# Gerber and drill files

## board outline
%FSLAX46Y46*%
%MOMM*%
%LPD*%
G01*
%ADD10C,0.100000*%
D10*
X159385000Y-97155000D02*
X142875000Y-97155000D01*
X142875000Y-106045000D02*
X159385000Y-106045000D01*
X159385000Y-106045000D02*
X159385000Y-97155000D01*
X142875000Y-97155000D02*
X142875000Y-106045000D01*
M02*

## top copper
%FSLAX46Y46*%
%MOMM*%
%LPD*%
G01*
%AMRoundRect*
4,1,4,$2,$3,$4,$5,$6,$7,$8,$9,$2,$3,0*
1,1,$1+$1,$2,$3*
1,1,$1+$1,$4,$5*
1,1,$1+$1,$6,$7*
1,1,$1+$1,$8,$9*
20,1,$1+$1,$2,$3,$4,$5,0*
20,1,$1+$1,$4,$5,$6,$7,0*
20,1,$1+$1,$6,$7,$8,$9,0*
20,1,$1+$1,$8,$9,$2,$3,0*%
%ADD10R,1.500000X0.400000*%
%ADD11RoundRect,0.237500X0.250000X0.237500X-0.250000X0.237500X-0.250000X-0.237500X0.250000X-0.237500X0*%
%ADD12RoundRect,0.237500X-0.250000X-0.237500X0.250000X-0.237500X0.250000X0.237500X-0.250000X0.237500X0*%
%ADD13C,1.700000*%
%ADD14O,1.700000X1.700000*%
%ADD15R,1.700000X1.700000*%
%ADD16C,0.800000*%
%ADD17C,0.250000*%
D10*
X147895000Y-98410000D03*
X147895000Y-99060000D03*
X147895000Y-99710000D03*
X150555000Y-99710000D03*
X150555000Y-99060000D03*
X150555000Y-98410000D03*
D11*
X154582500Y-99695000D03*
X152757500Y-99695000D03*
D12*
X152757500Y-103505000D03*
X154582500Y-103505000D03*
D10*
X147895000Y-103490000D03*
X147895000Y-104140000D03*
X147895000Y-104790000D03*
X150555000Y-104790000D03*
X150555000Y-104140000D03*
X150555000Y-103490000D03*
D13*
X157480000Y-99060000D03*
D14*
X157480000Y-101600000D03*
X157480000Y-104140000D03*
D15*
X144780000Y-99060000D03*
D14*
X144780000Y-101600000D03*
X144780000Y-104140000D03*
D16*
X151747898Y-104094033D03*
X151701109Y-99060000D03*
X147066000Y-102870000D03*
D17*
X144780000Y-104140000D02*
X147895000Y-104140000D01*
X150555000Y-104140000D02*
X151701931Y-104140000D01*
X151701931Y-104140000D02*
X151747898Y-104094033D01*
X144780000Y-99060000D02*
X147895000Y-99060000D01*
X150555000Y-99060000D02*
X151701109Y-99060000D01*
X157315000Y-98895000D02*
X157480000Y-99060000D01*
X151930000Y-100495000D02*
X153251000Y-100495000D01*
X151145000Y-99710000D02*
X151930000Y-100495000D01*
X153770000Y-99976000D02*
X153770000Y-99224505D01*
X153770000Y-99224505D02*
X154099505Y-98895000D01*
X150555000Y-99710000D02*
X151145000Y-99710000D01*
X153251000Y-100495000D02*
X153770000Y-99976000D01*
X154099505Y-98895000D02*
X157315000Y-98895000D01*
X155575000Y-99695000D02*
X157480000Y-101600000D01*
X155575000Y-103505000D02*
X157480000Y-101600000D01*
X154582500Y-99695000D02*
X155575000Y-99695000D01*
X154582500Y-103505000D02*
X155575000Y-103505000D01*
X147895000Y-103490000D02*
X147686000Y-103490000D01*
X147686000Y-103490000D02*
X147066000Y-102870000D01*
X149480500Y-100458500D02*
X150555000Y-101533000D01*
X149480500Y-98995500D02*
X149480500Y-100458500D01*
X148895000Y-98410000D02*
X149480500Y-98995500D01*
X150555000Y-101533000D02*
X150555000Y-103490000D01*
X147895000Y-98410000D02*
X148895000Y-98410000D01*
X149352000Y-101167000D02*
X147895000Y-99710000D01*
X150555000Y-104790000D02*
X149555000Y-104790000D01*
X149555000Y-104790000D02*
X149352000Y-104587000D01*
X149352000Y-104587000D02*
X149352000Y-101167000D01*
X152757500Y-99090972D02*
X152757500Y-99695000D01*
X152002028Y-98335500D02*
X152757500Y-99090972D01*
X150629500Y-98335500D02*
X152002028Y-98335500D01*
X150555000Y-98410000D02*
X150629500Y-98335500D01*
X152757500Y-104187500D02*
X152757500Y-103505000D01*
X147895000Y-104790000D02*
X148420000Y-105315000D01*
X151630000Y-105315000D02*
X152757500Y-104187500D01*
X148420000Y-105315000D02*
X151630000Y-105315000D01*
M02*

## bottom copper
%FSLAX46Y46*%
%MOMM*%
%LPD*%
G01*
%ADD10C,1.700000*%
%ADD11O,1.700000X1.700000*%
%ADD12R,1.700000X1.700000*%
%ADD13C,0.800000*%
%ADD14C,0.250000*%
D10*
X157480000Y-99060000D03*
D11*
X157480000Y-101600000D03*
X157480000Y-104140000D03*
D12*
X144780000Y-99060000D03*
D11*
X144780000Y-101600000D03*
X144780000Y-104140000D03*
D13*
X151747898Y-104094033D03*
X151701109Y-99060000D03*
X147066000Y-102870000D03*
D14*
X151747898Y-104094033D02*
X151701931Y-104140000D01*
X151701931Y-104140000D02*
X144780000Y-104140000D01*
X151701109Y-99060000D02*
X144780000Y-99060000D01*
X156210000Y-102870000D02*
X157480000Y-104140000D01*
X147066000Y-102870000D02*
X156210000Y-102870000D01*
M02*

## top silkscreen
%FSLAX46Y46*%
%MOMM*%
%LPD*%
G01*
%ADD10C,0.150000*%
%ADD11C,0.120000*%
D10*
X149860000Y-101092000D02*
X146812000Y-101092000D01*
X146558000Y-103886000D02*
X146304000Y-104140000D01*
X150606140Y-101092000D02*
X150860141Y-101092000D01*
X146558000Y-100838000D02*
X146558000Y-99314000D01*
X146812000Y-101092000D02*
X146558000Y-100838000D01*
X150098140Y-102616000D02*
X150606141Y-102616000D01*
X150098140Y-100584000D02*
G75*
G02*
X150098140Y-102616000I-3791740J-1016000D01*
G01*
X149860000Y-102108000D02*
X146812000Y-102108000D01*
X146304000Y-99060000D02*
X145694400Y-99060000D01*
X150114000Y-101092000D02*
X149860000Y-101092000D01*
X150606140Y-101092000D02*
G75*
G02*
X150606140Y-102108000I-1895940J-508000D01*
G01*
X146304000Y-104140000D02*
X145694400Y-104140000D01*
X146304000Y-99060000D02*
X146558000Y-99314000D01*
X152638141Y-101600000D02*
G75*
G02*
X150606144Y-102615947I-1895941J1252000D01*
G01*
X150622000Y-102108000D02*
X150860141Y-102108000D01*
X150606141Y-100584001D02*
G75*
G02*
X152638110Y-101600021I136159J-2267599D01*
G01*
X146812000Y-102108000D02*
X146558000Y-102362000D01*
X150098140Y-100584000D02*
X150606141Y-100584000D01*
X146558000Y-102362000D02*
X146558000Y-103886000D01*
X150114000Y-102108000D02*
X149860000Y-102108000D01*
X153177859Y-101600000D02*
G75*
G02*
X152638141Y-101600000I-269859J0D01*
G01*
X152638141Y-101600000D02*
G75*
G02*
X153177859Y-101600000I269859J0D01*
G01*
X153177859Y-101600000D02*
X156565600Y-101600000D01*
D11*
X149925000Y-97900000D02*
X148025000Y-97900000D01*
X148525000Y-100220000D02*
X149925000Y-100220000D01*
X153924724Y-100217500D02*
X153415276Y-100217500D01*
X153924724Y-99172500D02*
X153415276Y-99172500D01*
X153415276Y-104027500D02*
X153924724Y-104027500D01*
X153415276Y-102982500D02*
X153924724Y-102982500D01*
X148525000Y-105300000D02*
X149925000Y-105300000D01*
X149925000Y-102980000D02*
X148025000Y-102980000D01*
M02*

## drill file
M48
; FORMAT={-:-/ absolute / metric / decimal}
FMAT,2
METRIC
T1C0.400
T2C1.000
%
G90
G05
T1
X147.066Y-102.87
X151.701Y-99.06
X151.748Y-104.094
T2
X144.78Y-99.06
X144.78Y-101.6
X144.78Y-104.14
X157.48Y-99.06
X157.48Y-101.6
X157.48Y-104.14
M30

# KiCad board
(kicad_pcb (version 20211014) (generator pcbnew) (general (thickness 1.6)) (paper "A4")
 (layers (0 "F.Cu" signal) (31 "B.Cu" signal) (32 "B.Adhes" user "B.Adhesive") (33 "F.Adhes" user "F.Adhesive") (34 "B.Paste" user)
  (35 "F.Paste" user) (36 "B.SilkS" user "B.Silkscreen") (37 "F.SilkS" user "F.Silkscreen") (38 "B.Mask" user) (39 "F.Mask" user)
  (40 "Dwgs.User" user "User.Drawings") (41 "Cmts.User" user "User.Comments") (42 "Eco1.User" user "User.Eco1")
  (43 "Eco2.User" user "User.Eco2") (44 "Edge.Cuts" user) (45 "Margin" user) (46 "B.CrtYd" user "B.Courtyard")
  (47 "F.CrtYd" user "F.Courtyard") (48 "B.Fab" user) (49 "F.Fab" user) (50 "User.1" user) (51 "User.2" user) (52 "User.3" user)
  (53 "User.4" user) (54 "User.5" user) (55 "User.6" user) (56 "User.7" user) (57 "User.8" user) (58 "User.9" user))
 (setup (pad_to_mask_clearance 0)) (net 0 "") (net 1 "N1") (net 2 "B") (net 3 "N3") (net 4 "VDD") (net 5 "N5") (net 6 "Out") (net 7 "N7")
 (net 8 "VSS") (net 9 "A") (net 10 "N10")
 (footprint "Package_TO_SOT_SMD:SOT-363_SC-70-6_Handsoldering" (layer "F.Cu") (at 149.225 99.06)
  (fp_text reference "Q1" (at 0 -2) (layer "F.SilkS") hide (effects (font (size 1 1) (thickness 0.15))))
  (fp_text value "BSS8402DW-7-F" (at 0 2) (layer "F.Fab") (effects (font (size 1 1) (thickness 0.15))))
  (fp_line (start 0.7 -1.16) (end -1.2 -1.16) (layer "F.SilkS") (width 0.12))
  (fp_line (start -0.7 1.16) (end 0.7 1.16) (layer "F.SilkS") (width 0.12))
  (pad "1" smd rect (at -1.33 -0.65) (size 1.5 0.4) (layers "F.Cu" "F.Paste" "F.Mask") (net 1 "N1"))
  (pad "2" smd rect (at -1.33 0) (size 1.5 0.4) (layers "F.Cu" "F.Paste" "F.Mask") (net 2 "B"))
  (pad "3" smd rect (at -1.33 0.65) (size 1.5 0.4) (layers "F.Cu" "F.Paste" "F.Mask") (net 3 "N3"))
  (pad "4" smd rect (at 1.33 0.65) (size 1.5 0.4) (layers "F.Cu" "F.Paste" "F.Mask") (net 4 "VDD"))
  (pad "5" smd rect (at 1.33 0) (size 1.5 0.4) (layers "F.Cu" "F.Paste" "F.Mask") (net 2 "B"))
  (pad "6" smd rect (at 1.33 -0.65) (size 1.5 0.4) (layers "F.Cu" "F.Paste" "F.Mask") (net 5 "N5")))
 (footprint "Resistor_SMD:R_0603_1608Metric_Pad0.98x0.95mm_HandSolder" (layer "F.Cu") (at 153.67 99.695 180)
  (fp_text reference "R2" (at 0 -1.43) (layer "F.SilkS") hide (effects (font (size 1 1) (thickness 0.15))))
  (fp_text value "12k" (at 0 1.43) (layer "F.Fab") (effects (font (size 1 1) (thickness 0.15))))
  (fp_line (start -0.254724 -0.5225) (end 0.254724 -0.5225) (layer "F.SilkS") (width 0.12))
  (fp_line (start -0.254724 0.5225) (end 0.254724 0.5225) (layer "F.SilkS") (width 0.12))
  (pad "1" smd roundrect (at -0.9125 0 180) (size 0.975 0.95) (layers "F.Cu" "F.Paste" "F.Mask") (roundrect_rratio 0.25) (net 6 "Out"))
  (pad "2" smd roundrect (at 0.9125 0 180) (size 0.975 0.95) (layers "F.Cu" "F.Paste" "F.Mask") (roundrect_rratio 0.25) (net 5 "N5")))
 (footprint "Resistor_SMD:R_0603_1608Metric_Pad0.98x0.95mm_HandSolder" (layer "F.Cu") (at 153.67 103.505)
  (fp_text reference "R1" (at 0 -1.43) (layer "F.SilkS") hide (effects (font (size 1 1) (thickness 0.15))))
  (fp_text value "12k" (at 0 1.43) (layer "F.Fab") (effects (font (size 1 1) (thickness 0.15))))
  (fp_line (start -0.254724 0.5225) (end 0.254724 0.5225) (layer "F.SilkS") (width 0.12))
  (fp_line (start -0.254724 -0.5225) (end 0.254724 -0.5225) (layer "F.SilkS") (width 0.12))
  (pad "1" smd roundrect (at -0.9125 0) (size 0.975 0.95) (layers "F.Cu" "F.Paste" "F.Mask") (roundrect_rratio 0.25) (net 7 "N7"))
  (pad "2" smd roundrect (at 0.9125 0) (size 0.975 0.95) (layers "F.Cu" "F.Paste" "F.Mask") (roundrect_rratio 0.25) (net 6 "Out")))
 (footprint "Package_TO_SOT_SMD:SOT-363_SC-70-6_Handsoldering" (layer "F.Cu") (at 149.225 104.14)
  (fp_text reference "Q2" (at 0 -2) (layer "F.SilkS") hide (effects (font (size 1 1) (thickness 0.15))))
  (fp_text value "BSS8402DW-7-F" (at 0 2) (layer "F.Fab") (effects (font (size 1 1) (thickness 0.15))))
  (fp_line (start -0.7 1.16) (end 0.7 1.16) (layer "F.SilkS") (width 0.12))
  (fp_line (start 0.7 -1.16) (end -1.2 -1.16) (layer "F.SilkS") (width 0.12))
  (pad "1" smd rect (at -1.33 -0.65) (size 1.5 0.4) (layers "F.Cu" "F.Paste" "F.Mask") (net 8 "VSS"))
  (pad "2" smd rect (at -1.33 0) (size 1.5 0.4) (layers "F.Cu" "F.Paste" "F.Mask") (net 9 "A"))
  (pad "3" smd rect (at -1.33 0.65) (size 1.5 0.4) (layers "F.Cu" "F.Paste" "F.Mask") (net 7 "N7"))
  (pad "4" smd rect (at 1.33 0.65) (size 1.5 0.4) (layers "F.Cu" "F.Paste" "F.Mask") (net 3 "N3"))
  (pad "5" smd rect (at 1.33 0) (size 1.5 0.4) (layers "F.Cu" "F.Paste" "F.Mask") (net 9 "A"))
  (pad "6" smd rect (at 1.33 -0.65) (size 1.5 0.4) (layers "F.Cu" "F.Paste" "F.Mask") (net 1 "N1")))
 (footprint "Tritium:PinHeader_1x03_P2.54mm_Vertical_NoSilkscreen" (layer "F.Cu") (at 157.48 99.06)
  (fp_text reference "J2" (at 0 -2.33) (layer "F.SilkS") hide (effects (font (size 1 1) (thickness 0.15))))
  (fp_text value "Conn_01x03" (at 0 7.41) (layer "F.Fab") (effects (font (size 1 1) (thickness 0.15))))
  (pad "1" thru_hole circle (at 0 0) (size 1.7 1.7) (drill 1) (layers *.Cu *.Mask) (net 4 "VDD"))
  (pad "2" thru_hole oval (at 0 2.54) (size 1.7 1.7) (drill 1) (layers *.Cu *.Mask) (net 6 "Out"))
  (pad "3" thru_hole oval (at 0 5.08) (size 1.7 1.7) (drill 1) (layers *.Cu *.Mask) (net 8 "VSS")))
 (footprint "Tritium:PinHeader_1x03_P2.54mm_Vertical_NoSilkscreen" (layer "F.Cu") (at 144.78 99.06)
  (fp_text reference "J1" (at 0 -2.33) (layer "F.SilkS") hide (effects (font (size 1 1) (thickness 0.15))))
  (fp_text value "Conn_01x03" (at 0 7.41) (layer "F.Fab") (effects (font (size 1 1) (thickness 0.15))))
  (pad "1" thru_hole rect (at 0 0) (size 1.7 1.7) (drill 1) (layers *.Cu *.Mask) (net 2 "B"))
  (pad "2" thru_hole oval (at 0 2.54) (size 1.7 1.7) (drill 1) (layers *.Cu *.Mask) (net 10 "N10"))
  (pad "3" thru_hole oval (at 0 5.08) (size 1.7 1.7) (drill 1) (layers *.Cu *.Mask) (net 9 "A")))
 (gr_line (start 149.86 101.092) (end 146.812 101.092) (layer "F.SilkS") (width 0.15))
 (gr_line (start 146.558 103.886) (end 146.304 104.14) (layer "F.SilkS") (width 0.15))
 (gr_line (start 150.60614 101.092) (end 150.860141 101.092) (layer "F.SilkS") (width 0.15))
 (gr_line (start 146.558 100.838) (end 146.558 99.314) (layer "F.SilkS") (width 0.15))
 (gr_line (start 146.812 101.092) (end 146.558 100.838) (layer "F.SilkS") (width 0.15))
 (gr_line (start 150.09814 102.616) (end 150.606141 102.616) (layer "F.SilkS") (width 0.15))
 (gr_arc (start 150.09814 100.584) (mid 150.2319 101.6) (end 150.09814 102.616) (layer "F.SilkS") (width 0.15))
 (gr_line (start 149.86 102.108) (end 146.812 102.108) (layer "F.SilkS") (width 0.15))
 (gr_line (start 146.304 99.06) (end 145.6944 99.06) (layer "F.SilkS") (width 0.15))
 (gr_line (start 150.114 101.092) (end 149.86 101.092) (layer "F.SilkS") (width 0.15))
 (gr_arc (start 150.60614 101.092) (mid 150.673017 101.6) (end 150.60614 102.108) (layer "F.SilkS") (width 0.15))
 (gr_line (start 146.304 104.14) (end 145.6944 104.14) (layer "F.SilkS") (width 0.15))
 (gr_line (start 146.304 99.06) (end 146.558 99.314) (layer "F.SilkS") (width 0.15))
 (gr_arc (start 152.638141 101.6) (mid 151.758253 102.380208) (end 150.606141 102.616) (layer "F.SilkS") (width 0.15))
 (gr_line (start 150.622 102.108) (end 150.860141 102.108) (layer "F.SilkS") (width 0.15))
 (gr_arc (start 150.606141 100.584001) (mid 151.758276 100.819746) (end 152.638141 101.6) (layer "F.SilkS") (width 0.15))
 (gr_line (start 146.812 102.108) (end 146.558 102.362) (layer "F.SilkS") (width 0.15))
 (gr_line (start 150.09814 100.584) (end 150.606141 100.584) (layer "F.SilkS") (width 0.15))
 (gr_line (start 146.558 102.362) (end 146.558 103.886) (layer "F.SilkS") (width 0.15))
 (gr_line (start 150.114 102.108) (end 149.86 102.108) (layer "F.SilkS") (width 0.15))
 (gr_circle (center 152.908 101.6) (end 152.638141 101.6) (layer "F.SilkS") (width 0.15) (fill none))
 (gr_line (start 153.177859 101.6) (end 156.5656 101.6) (layer "F.SilkS") (width 0.15))
 (gr_line (start 159.385 97.155) (end 142.875 97.155) (layer "Edge.Cuts") (width 0.1))
 (gr_line (start 142.875 106.045) (end 159.385 106.045) (layer "Edge.Cuts") (width 0.1))
 (gr_line (start 159.385 106.045) (end 159.385 97.155) (layer "Edge.Cuts") (width 0.1))
 (gr_line (start 142.875 97.155) (end 142.875 106.045) (layer "Edge.Cuts") (width 0.1))
 (segment (start 144.78 104.14) (end 147.895 104.14) (width 0.25) (layer "F.Cu") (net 9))
 (segment (start 150.555 104.14) (end 151.701931 104.14) (width 0.25) (layer "F.Cu") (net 9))
 (segment (start 151.701931 104.14) (end 151.747898 104.094033) (width 0.25) (layer "F.Cu") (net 9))
 (via (at 151.747898 104.094033) (size 0.8) (drill 0.4) (layers "F.Cu" "B.Cu") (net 9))
 (segment (start 151.747898 104.094033) (end 151.701931 104.14) (width 0.25) (layer "B.Cu") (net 9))
 (segment (start 151.701931 104.14) (end 144.78 104.14) (width 0.25) (layer "B.Cu") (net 9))
 (segment (start 144.78 99.06) (end 147.895 99.06) (width 0.25) (layer "F.Cu") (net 2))
 (segment (start 150.555 99.06) (end 151.701109 99.06) (width 0.25) (layer "F.Cu") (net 2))
 (via (at 151.701109 99.06) (size 0.8) (drill 0.4) (layers "F.Cu" "B.Cu") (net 2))
 (segment (start 151.701109 99.06) (end 144.78 99.06) (width 0.25) (layer "B.Cu") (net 2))
 (segment (start 157.315 98.895) (end 157.48 99.06) (width 0.25) (layer "F.Cu") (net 4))
 (segment (start 151.93 100.495) (end 153.251 100.495) (width 0.25) (layer "F.Cu") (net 4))
 (segment (start 151.145 99.71) (end 151.93 100.495) (width 0.25) (layer "F.Cu") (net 4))
 (segment (start 153.77 99.976) (end 153.77 99.224505) (width 0.25) (layer "F.Cu") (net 4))
 (segment (start 153.77 99.224505) (end 154.099505 98.895) (width 0.25) (layer "F.Cu") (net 4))
 (segment (start 150.555 99.71) (end 151.145 99.71) (width 0.25) (layer "F.Cu") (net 4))
 (segment (start 153.251 100.495) (end 153.77 99.976) (width 0.25) (layer "F.Cu") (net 4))
 (segment (start 154.099505 98.895) (end 157.315 98.895) (width 0.25) (layer "F.Cu") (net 4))
 (segment (start 155.575 99.695) (end 157.48 101.6) (width 0.25) (layer "F.Cu") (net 6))
 (segment (start 155.575 103.505) (end 157.48 101.6) (width 0.25) (layer "F.Cu") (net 6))
 (segment (start 154.5825 99.695) (end 155.575 99.695) (width 0.25) (layer "F.Cu") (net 6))
 (segment (start 154.5825 103.505) (end 155.575 103.505) (width 0.25) (layer "F.Cu") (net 6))
 (segment (start 147.895 103.49) (end 147.686 103.49) (width 0.25) (layer "F.Cu") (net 8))
 (segment (start 147.686 103.49) (end 147.066 102.87) (width 0.25) (layer "F.Cu") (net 8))
 (via (at 147.066 102.87) (size 0.8) (drill 0.4) (layers "F.Cu" "B.Cu") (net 8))
 (segment (start 156.21 102.87) (end 157.48 104.14) (width 0.25) (layer "B.Cu") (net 8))
 (segment (start 147.066 102.87) (end 156.21 102.87) (width 0.25) (layer "B.Cu") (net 8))
 (segment (start 149.4805 100.4585) (end 150.555 101.533) (width 0.25) (layer "F.Cu") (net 1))
 (segment (start 149.4805 98.9955) (end 149.4805 100.4585) (width 0.25) (layer "F.Cu") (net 1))
 (segment (start 148.895 98.41) (end 149.4805 98.9955) (width 0.25) (layer "F.Cu") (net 1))
 (segment (start 150.555 101.533) (end 150.555 103.49) (width 0.25) (layer "F.Cu") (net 1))
 (segment (start 147.895 98.41) (end 148.895 98.41) (width 0.25) (layer "F.Cu") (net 1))
 (segment (start 149.352 101.167) (end 147.895 99.71) (width 0.25) (layer "F.Cu") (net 3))
 (segment (start 150.555 104.79) (end 149.555 104.79) (width 0.25) (layer "F.Cu") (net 3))
 (segment (start 149.555 104.79) (end 149.352 104.587) (width 0.25) (layer "F.Cu") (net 3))
 (segment (start 149.352 104.587) (end 149.352 101.167) (width 0.25) (layer "F.Cu") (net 3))
 (segment (start 152.7575 99.090972) (end 152.7575 99.695) (width 0.25) (layer "F.Cu") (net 5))
 (segment (start 152.002028 98.3355) (end 152.7575 99.090972) (width 0.25) (layer "F.Cu") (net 5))
 (segment (start 150.6295 98.3355) (end 152.002028 98.3355) (width 0.25) (layer "F.Cu") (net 5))
 (segment (start 150.555 98.41) (end 150.6295 98.3355) (width 0.25) (layer "F.Cu") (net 5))
 (segment (start 152.7575 104.1875) (end 152.7575 103.505) (width 0.25) (layer "F.Cu") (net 7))
 (segment (start 147.895 104.79) (end 148.42 105.315) (width 0.25) (layer "F.Cu") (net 7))
 (segment (start 151.63 105.315) (end 152.7575 104.1875) (width 0.25) (layer "F.Cu") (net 7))
 (segment (start 148.42 105.315) (end 151.63 105.315) (width 0.25) (layer "F.Cu") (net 7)))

